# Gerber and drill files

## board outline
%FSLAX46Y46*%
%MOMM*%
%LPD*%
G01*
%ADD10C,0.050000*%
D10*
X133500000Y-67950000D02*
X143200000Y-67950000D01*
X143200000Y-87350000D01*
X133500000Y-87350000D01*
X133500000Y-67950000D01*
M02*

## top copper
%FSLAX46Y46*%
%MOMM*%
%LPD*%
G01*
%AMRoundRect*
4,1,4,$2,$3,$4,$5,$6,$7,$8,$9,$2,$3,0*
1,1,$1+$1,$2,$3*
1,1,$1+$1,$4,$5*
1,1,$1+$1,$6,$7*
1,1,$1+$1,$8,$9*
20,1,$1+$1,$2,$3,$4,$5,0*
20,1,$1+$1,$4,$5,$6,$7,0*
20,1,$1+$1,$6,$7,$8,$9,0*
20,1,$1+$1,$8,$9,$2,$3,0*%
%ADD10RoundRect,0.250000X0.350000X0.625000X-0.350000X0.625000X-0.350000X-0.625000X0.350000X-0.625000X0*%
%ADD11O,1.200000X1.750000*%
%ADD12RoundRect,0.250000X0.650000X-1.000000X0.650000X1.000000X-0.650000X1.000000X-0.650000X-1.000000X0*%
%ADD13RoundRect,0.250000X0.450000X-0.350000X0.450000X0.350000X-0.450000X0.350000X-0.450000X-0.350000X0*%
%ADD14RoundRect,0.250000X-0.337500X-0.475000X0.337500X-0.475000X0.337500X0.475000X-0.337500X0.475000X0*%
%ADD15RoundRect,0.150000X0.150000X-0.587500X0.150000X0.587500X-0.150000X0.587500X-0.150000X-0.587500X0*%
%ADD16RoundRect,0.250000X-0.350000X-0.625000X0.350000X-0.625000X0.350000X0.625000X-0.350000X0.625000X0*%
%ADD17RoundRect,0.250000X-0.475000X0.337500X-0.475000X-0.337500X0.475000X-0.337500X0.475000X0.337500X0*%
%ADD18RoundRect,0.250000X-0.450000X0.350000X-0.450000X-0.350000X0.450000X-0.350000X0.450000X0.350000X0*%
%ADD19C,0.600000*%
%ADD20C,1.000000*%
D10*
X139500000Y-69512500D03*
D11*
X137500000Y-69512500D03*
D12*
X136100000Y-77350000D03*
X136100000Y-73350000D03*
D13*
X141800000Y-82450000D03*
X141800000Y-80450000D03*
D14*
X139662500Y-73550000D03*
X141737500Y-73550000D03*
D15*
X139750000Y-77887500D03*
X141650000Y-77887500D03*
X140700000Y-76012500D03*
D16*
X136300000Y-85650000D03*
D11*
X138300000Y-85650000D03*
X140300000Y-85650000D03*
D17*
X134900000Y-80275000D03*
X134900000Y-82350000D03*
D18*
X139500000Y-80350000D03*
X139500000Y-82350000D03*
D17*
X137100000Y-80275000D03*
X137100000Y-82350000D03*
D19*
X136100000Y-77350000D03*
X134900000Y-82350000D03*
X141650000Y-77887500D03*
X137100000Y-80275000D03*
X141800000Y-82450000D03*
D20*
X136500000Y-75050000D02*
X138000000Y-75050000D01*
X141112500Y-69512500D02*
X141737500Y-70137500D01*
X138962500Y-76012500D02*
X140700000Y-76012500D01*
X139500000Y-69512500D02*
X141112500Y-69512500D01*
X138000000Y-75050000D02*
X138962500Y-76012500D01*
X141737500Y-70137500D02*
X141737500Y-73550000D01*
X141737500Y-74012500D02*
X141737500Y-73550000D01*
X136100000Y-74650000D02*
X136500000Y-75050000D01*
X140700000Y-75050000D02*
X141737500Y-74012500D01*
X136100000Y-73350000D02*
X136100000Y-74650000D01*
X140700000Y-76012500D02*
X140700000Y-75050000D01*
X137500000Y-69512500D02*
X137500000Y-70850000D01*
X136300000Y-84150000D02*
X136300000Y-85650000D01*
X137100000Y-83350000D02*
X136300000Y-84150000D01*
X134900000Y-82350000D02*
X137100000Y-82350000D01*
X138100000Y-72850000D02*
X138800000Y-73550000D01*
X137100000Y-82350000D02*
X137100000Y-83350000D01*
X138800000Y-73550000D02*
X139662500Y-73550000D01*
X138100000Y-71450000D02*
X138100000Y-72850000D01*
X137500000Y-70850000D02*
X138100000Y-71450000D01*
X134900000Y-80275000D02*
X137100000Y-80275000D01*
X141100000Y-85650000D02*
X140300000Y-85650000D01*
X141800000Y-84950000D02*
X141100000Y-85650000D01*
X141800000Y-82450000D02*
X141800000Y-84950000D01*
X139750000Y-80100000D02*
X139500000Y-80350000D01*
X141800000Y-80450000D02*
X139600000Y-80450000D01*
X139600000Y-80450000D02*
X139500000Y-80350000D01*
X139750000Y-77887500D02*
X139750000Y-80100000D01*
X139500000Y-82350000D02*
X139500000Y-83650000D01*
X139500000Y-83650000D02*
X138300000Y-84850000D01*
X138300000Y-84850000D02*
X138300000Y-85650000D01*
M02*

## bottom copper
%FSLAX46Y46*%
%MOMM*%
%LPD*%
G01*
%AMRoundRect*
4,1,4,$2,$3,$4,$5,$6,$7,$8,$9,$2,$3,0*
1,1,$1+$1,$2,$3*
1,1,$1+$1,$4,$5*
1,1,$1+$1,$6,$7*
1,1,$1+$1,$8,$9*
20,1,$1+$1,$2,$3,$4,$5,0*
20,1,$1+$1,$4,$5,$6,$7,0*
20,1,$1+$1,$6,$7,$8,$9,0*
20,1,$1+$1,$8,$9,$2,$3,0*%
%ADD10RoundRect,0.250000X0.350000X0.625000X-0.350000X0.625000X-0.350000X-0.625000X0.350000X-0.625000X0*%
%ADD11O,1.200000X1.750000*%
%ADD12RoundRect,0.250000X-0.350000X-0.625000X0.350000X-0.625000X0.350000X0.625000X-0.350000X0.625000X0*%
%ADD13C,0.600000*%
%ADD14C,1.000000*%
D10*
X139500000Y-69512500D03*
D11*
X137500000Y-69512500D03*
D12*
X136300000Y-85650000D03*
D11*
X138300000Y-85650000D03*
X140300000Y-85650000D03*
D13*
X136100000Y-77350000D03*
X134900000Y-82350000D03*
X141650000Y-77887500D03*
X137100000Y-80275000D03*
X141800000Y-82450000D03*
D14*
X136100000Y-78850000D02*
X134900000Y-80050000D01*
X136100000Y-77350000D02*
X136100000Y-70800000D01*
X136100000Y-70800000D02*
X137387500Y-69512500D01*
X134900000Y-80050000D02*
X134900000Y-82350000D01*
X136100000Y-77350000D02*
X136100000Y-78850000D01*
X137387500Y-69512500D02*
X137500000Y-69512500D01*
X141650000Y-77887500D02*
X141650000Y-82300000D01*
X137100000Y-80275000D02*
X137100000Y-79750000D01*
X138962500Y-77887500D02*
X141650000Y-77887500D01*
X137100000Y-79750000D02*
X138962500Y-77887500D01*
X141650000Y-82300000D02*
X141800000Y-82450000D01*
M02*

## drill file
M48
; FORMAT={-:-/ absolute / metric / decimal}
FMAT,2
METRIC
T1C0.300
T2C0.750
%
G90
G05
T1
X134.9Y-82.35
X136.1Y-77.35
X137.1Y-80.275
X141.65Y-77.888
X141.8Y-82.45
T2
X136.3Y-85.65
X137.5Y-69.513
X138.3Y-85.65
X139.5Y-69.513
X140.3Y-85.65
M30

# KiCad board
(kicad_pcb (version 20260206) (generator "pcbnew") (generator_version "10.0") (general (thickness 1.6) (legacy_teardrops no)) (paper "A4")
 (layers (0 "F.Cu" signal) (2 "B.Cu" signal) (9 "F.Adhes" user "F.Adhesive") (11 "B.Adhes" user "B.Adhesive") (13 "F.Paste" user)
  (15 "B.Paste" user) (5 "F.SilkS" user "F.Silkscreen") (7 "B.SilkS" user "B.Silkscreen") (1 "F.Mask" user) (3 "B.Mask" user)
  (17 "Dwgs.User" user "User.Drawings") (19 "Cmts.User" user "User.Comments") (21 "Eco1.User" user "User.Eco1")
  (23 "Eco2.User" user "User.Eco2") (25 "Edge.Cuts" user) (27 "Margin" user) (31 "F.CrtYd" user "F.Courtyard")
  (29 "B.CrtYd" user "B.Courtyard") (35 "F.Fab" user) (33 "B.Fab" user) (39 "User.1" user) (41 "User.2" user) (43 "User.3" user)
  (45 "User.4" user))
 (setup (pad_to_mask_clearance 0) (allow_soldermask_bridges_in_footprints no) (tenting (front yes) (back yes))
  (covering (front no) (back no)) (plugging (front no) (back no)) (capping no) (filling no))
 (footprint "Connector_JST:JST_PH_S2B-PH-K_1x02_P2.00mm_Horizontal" (layer "F.Cu") (at 139.5 69.5125 180)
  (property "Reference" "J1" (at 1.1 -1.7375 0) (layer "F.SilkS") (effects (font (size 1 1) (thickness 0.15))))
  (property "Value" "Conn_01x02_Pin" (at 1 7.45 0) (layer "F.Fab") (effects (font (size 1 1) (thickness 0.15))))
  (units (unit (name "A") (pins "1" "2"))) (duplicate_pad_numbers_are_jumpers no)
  (pad "1" thru_hole roundrect (at 0 0 180) (size 1.2 1.75) (drill 0.75) (layers "*.Cu" "*.Mask") (remove_unused_layers no)
   (roundrect_rratio 0.208333) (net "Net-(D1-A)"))
  (pad "2" thru_hole oval (at 2 0 180) (size 1.2 1.75) (drill 0.75) (layers "*.Cu" "*.Mask") (remove_unused_layers no) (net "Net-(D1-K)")))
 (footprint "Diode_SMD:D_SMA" (layer "F.Cu") (at 136.1 75.35 90)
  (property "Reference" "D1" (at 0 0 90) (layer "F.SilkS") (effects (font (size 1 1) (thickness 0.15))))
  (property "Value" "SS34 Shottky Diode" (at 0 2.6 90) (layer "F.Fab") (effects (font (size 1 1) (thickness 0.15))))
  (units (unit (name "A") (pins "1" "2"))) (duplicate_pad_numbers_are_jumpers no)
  (pad "1" smd roundrect (at -2 0 90) (size 2.5 1.8) (layers "F.Cu" "F.Mask" "F.Paste") (roundrect_rratio 0.1388888889) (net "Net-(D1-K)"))
  (pad "2" smd roundrect (at 2 0 90) (size 2.5 1.8) (layers "F.Cu" "F.Mask" "F.Paste") (roundrect_rratio 0.1388888889) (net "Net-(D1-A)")))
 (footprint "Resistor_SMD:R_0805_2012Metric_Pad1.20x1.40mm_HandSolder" (layer "F.Cu") (at 141.8 81.45 90)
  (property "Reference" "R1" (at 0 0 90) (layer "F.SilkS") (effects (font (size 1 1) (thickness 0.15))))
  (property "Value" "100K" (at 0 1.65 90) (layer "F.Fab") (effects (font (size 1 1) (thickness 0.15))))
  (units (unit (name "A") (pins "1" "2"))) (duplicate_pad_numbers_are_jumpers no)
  (pad "1" smd roundrect (at -1 0 90) (size 1.2 1.4) (layers "F.Cu" "F.Mask" "F.Paste") (roundrect_rratio 0.208333) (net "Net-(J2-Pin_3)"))
  (pad "2" smd roundrect (at 1 0 90) (size 1.2 1.4) (layers "F.Cu" "F.Mask" "F.Paste") (roundrect_rratio 0.208333) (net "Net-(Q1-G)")))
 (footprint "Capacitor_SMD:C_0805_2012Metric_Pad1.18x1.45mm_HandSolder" (layer "F.Cu") (at 140.7 73.55)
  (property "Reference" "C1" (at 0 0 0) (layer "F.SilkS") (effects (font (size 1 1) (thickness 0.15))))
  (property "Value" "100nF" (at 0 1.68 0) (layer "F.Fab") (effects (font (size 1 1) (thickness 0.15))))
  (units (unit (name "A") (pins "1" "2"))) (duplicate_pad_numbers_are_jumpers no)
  (pad "1" smd roundrect (at -1.0375 0) (size 1.175 1.45) (layers "F.Cu" "F.Mask" "F.Paste") (roundrect_rratio 0.212766) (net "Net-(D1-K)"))
  (pad "2" smd roundrect (at 1.0375 0) (size 1.175 1.45) (layers "F.Cu" "F.Mask" "F.Paste") (roundrect_rratio 0.212766) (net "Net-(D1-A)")))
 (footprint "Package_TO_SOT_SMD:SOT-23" (layer "F.Cu") (at 140.7 76.95 90)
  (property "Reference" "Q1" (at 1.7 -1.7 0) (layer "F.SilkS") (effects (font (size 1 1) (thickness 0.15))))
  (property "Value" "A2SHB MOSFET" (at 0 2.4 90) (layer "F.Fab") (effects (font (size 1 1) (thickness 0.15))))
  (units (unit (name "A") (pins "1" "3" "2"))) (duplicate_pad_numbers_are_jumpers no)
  (pad "1" smd roundrect (at -0.9375 -0.95 90) (size 1.475 0.6) (layers "F.Cu" "F.Mask" "F.Paste") (roundrect_rratio 0.25)
   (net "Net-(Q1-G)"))
  (pad "2" smd roundrect (at -0.9375 0.95 90) (size 1.475 0.6) (layers "F.Cu" "F.Mask" "F.Paste") (roundrect_rratio 0.25)
   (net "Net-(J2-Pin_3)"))
  (pad "3" smd roundrect (at 0.9375 0 90) (size 1.475 0.6) (layers "F.Cu" "F.Mask" "F.Paste") (roundrect_rratio 0.25) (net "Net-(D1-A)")))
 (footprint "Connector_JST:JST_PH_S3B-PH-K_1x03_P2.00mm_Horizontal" (layer "F.Cu") (at 136.3 85.65)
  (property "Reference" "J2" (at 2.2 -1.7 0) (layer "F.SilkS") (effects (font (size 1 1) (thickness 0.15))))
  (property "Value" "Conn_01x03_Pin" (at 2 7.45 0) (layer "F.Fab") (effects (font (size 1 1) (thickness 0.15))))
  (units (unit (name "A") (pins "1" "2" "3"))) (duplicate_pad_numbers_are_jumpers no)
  (pad "1" thru_hole roundrect (at 0 0) (size 1.2 1.75) (drill 0.75) (layers "*.Cu" "*.Mask") (remove_unused_layers no)
   (roundrect_rratio 0.208333) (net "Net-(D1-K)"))
  (pad "2" thru_hole oval (at 2 0) (size 1.2 1.75) (drill 0.75) (layers "*.Cu" "*.Mask") (remove_unused_layers no) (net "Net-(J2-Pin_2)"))
  (pad "3" thru_hole oval (at 4 0) (size 1.2 1.75) (drill 0.75) (layers "*.Cu" "*.Mask") (remove_unused_layers no) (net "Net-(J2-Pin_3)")))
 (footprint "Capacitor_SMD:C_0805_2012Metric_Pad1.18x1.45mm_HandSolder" (layer "F.Cu") (at 134.9 81.3125 -90)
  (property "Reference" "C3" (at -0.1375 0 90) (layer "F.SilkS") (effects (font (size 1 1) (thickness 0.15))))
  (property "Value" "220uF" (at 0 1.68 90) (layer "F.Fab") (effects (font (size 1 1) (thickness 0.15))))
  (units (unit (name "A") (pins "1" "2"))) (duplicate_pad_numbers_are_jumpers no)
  (pad "1" smd roundrect (at -1.0375 0 270) (size 1.175 1.45) (layers "F.Cu" "F.Mask" "F.Paste") (roundrect_rratio 0.212766)
   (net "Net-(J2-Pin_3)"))
  (pad "2" smd roundrect (at 1.0375 0 270) (size 1.175 1.45) (layers "F.Cu" "F.Mask" "F.Paste") (roundrect_rratio 0.212766)
   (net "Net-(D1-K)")))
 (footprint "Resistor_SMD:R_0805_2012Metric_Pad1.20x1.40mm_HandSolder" (layer "F.Cu") (at 139.5 81.35 -90)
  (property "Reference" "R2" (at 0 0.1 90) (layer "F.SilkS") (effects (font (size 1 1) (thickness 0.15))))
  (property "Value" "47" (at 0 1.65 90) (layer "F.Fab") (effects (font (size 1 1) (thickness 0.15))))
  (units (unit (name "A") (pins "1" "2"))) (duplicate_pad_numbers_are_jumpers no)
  (pad "1" smd roundrect (at -1 0 270) (size 1.2 1.4) (layers "F.Cu" "F.Mask" "F.Paste") (roundrect_rratio 0.208333) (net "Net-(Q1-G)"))
  (pad "2" smd roundrect (at 1 0 270) (size 1.2 1.4) (layers "F.Cu" "F.Mask" "F.Paste") (roundrect_rratio 0.208333) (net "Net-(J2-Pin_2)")))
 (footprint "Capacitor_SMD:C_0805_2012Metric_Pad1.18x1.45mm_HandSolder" (layer "F.Cu") (at 137.1 81.3125 -90)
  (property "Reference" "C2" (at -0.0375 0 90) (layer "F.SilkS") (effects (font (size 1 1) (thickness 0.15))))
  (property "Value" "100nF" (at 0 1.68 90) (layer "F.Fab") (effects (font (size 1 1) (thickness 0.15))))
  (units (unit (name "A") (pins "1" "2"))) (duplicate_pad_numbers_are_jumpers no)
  (pad "1" smd roundrect (at -1.0375 0 270) (size 1.175 1.45) (layers "F.Cu" "F.Mask" "F.Paste") (roundrect_rratio 0.212766)
   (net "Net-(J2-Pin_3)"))
  (pad "2" smd roundrect (at 1.0375 0 270) (size 1.175 1.45) (layers "F.Cu" "F.Mask" "F.Paste") (roundrect_rratio 0.212766)
   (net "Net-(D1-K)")))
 (gr_rect (start 133.5 67.95) (end 143.2 87.35) (stroke (width 0.05) (type default)) (fill no) (layer "Edge.Cuts"))
 (segment (start 136.5 75.05) (end 138 75.05) (width 1) (layer "F.Cu") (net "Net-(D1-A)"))
 (segment (start 141.1125 69.5125) (end 141.7375 70.1375) (width 1) (layer "F.Cu") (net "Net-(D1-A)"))
 (segment (start 138.9625 76.0125) (end 140.7 76.0125) (width 1) (layer "F.Cu") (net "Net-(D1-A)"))
 (segment (start 139.5 69.5125) (end 141.1125 69.5125) (width 1) (layer "F.Cu") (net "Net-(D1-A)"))
 (segment (start 138 75.05) (end 138.9625 76.0125) (width 1) (layer "F.Cu") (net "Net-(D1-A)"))
 (segment (start 141.7375 70.1375) (end 141.7375 73.55) (width 1) (layer "F.Cu") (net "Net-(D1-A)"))
 (segment (start 141.7375 74.0125) (end 141.7375 73.55) (width 1) (layer "F.Cu") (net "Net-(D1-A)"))
 (segment (start 136.1 74.65) (end 136.5 75.05) (width 1) (layer "F.Cu") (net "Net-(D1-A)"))
 (segment (start 140.7 75.05) (end 141.7375 74.0125) (width 1) (layer "F.Cu") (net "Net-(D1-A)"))
 (segment (start 136.1 73.35) (end 136.1 74.65) (width 1) (layer "F.Cu") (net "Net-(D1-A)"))
 (segment (start 140.7 76.0125) (end 140.7 75.05) (width 1) (layer "F.Cu") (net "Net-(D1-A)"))
 (segment (start 137.5 69.5125) (end 137.5 70.85) (width 1) (layer "F.Cu") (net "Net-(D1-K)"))
 (segment (start 136.3 84.15) (end 136.3 85.65) (width 1) (layer "F.Cu") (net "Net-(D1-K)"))
 (segment (start 137.1 83.35) (end 136.3 84.15) (width 1) (layer "F.Cu") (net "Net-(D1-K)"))
 (segment (start 134.9 82.35) (end 137.1 82.35) (width 1) (layer "F.Cu") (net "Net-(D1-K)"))
 (segment (start 138.1 72.85) (end 138.8 73.55) (width 1) (layer "F.Cu") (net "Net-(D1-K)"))
 (segment (start 137.1 82.35) (end 137.1 83.35) (width 1) (layer "F.Cu") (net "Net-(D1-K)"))
 (segment (start 138.8 73.55) (end 139.6625 73.55) (width 1) (layer "F.Cu") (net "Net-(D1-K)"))
 (segment (start 138.1 71.45) (end 138.1 72.85) (width 1) (layer "F.Cu") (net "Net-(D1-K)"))
 (segment (start 137.5 70.85) (end 138.1 71.45) (width 1) (layer "F.Cu") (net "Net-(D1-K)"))
 (via (at 136.1 77.35) (size 0.6) (drill 0.3) (layers "F.Cu" "B.Cu") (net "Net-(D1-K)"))
 (via (at 134.9 82.35) (size 0.6) (drill 0.3) (layers "F.Cu" "B.Cu") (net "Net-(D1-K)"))
 (segment (start 136.1 78.85) (end 134.9 80.05) (width 1) (layer "B.Cu") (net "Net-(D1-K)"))
 (segment (start 136.1 77.35) (end 136.1 70.8) (width 1) (layer "B.Cu") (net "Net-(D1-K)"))
 (segment (start 136.1 70.8) (end 137.3875 69.5125) (width 1) (layer "B.Cu") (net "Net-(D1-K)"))
 (segment (start 134.9 80.05) (end 134.9 82.35) (width 1) (layer "B.Cu") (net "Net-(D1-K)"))
 (segment (start 136.1 77.35) (end 136.1 78.85) (width 1) (layer "B.Cu") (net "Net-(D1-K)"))
 (segment (start 137.3875 69.5125) (end 137.5 69.5125) (width 1) (layer "B.Cu") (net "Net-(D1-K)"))
 (segment (start 134.9 80.275) (end 137.1 80.275) (width 1) (layer "F.Cu") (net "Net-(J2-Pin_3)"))
 (segment (start 141.1 85.65) (end 140.3 85.65) (width 1) (layer "F.Cu") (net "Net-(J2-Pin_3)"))
 (segment (start 141.8 84.95) (end 141.1 85.65) (width 1) (layer "F.Cu") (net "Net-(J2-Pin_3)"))
 (segment (start 141.8 82.45) (end 141.8 84.95) (width 1) (layer "F.Cu") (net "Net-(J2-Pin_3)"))
 (via (at 141.65 77.8875) (size 0.6) (drill 0.3) (layers "F.Cu" "B.Cu") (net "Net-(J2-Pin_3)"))
 (via (at 137.1 80.275) (size 0.6) (drill 0.3) (layers "F.Cu" "B.Cu") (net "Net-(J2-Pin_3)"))
 (via (at 141.8 82.45) (size 0.6) (drill 0.3) (layers "F.Cu" "B.Cu") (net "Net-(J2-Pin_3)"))
 (segment (start 141.65 77.8875) (end 141.65 82.3) (width 1) (layer "B.Cu") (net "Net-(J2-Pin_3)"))
 (segment (start 137.1 80.275) (end 137.1 79.75) (width 1) (layer "B.Cu") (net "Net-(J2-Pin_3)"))
 (segment (start 138.9625 77.8875) (end 141.65 77.8875) (width 1) (layer "B.Cu") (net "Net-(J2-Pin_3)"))
 (segment (start 137.1 79.75) (end 138.9625 77.8875) (width 1) (layer "B.Cu") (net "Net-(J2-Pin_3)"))
 (segment (start 141.65 82.3) (end 141.8 82.45) (width 1) (layer "B.Cu") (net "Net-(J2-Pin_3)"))
 (segment (start 139.75 80.1) (end 139.5 80.35) (width 1) (layer "F.Cu") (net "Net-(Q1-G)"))
 (segment (start 141.8 80.45) (end 139.6 80.45) (width 1) (layer "F.Cu") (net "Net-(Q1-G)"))
 (segment (start 139.6 80.45) (end 139.5 80.35) (width 1) (layer "F.Cu") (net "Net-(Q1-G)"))
 (segment (start 139.75 77.8875) (end 139.75 80.1) (width 1) (layer "F.Cu") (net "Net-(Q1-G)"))
 (segment (start 139.5 82.35) (end 139.5 83.65) (width 1) (layer "F.Cu") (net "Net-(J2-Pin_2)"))
 (segment (start 139.5 83.65) (end 138.3 84.85) (width 1) (layer "F.Cu") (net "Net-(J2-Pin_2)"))
 (segment (start 138.3 84.85) (end 138.3 85.65) (width 1) (layer "F.Cu") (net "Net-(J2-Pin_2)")))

